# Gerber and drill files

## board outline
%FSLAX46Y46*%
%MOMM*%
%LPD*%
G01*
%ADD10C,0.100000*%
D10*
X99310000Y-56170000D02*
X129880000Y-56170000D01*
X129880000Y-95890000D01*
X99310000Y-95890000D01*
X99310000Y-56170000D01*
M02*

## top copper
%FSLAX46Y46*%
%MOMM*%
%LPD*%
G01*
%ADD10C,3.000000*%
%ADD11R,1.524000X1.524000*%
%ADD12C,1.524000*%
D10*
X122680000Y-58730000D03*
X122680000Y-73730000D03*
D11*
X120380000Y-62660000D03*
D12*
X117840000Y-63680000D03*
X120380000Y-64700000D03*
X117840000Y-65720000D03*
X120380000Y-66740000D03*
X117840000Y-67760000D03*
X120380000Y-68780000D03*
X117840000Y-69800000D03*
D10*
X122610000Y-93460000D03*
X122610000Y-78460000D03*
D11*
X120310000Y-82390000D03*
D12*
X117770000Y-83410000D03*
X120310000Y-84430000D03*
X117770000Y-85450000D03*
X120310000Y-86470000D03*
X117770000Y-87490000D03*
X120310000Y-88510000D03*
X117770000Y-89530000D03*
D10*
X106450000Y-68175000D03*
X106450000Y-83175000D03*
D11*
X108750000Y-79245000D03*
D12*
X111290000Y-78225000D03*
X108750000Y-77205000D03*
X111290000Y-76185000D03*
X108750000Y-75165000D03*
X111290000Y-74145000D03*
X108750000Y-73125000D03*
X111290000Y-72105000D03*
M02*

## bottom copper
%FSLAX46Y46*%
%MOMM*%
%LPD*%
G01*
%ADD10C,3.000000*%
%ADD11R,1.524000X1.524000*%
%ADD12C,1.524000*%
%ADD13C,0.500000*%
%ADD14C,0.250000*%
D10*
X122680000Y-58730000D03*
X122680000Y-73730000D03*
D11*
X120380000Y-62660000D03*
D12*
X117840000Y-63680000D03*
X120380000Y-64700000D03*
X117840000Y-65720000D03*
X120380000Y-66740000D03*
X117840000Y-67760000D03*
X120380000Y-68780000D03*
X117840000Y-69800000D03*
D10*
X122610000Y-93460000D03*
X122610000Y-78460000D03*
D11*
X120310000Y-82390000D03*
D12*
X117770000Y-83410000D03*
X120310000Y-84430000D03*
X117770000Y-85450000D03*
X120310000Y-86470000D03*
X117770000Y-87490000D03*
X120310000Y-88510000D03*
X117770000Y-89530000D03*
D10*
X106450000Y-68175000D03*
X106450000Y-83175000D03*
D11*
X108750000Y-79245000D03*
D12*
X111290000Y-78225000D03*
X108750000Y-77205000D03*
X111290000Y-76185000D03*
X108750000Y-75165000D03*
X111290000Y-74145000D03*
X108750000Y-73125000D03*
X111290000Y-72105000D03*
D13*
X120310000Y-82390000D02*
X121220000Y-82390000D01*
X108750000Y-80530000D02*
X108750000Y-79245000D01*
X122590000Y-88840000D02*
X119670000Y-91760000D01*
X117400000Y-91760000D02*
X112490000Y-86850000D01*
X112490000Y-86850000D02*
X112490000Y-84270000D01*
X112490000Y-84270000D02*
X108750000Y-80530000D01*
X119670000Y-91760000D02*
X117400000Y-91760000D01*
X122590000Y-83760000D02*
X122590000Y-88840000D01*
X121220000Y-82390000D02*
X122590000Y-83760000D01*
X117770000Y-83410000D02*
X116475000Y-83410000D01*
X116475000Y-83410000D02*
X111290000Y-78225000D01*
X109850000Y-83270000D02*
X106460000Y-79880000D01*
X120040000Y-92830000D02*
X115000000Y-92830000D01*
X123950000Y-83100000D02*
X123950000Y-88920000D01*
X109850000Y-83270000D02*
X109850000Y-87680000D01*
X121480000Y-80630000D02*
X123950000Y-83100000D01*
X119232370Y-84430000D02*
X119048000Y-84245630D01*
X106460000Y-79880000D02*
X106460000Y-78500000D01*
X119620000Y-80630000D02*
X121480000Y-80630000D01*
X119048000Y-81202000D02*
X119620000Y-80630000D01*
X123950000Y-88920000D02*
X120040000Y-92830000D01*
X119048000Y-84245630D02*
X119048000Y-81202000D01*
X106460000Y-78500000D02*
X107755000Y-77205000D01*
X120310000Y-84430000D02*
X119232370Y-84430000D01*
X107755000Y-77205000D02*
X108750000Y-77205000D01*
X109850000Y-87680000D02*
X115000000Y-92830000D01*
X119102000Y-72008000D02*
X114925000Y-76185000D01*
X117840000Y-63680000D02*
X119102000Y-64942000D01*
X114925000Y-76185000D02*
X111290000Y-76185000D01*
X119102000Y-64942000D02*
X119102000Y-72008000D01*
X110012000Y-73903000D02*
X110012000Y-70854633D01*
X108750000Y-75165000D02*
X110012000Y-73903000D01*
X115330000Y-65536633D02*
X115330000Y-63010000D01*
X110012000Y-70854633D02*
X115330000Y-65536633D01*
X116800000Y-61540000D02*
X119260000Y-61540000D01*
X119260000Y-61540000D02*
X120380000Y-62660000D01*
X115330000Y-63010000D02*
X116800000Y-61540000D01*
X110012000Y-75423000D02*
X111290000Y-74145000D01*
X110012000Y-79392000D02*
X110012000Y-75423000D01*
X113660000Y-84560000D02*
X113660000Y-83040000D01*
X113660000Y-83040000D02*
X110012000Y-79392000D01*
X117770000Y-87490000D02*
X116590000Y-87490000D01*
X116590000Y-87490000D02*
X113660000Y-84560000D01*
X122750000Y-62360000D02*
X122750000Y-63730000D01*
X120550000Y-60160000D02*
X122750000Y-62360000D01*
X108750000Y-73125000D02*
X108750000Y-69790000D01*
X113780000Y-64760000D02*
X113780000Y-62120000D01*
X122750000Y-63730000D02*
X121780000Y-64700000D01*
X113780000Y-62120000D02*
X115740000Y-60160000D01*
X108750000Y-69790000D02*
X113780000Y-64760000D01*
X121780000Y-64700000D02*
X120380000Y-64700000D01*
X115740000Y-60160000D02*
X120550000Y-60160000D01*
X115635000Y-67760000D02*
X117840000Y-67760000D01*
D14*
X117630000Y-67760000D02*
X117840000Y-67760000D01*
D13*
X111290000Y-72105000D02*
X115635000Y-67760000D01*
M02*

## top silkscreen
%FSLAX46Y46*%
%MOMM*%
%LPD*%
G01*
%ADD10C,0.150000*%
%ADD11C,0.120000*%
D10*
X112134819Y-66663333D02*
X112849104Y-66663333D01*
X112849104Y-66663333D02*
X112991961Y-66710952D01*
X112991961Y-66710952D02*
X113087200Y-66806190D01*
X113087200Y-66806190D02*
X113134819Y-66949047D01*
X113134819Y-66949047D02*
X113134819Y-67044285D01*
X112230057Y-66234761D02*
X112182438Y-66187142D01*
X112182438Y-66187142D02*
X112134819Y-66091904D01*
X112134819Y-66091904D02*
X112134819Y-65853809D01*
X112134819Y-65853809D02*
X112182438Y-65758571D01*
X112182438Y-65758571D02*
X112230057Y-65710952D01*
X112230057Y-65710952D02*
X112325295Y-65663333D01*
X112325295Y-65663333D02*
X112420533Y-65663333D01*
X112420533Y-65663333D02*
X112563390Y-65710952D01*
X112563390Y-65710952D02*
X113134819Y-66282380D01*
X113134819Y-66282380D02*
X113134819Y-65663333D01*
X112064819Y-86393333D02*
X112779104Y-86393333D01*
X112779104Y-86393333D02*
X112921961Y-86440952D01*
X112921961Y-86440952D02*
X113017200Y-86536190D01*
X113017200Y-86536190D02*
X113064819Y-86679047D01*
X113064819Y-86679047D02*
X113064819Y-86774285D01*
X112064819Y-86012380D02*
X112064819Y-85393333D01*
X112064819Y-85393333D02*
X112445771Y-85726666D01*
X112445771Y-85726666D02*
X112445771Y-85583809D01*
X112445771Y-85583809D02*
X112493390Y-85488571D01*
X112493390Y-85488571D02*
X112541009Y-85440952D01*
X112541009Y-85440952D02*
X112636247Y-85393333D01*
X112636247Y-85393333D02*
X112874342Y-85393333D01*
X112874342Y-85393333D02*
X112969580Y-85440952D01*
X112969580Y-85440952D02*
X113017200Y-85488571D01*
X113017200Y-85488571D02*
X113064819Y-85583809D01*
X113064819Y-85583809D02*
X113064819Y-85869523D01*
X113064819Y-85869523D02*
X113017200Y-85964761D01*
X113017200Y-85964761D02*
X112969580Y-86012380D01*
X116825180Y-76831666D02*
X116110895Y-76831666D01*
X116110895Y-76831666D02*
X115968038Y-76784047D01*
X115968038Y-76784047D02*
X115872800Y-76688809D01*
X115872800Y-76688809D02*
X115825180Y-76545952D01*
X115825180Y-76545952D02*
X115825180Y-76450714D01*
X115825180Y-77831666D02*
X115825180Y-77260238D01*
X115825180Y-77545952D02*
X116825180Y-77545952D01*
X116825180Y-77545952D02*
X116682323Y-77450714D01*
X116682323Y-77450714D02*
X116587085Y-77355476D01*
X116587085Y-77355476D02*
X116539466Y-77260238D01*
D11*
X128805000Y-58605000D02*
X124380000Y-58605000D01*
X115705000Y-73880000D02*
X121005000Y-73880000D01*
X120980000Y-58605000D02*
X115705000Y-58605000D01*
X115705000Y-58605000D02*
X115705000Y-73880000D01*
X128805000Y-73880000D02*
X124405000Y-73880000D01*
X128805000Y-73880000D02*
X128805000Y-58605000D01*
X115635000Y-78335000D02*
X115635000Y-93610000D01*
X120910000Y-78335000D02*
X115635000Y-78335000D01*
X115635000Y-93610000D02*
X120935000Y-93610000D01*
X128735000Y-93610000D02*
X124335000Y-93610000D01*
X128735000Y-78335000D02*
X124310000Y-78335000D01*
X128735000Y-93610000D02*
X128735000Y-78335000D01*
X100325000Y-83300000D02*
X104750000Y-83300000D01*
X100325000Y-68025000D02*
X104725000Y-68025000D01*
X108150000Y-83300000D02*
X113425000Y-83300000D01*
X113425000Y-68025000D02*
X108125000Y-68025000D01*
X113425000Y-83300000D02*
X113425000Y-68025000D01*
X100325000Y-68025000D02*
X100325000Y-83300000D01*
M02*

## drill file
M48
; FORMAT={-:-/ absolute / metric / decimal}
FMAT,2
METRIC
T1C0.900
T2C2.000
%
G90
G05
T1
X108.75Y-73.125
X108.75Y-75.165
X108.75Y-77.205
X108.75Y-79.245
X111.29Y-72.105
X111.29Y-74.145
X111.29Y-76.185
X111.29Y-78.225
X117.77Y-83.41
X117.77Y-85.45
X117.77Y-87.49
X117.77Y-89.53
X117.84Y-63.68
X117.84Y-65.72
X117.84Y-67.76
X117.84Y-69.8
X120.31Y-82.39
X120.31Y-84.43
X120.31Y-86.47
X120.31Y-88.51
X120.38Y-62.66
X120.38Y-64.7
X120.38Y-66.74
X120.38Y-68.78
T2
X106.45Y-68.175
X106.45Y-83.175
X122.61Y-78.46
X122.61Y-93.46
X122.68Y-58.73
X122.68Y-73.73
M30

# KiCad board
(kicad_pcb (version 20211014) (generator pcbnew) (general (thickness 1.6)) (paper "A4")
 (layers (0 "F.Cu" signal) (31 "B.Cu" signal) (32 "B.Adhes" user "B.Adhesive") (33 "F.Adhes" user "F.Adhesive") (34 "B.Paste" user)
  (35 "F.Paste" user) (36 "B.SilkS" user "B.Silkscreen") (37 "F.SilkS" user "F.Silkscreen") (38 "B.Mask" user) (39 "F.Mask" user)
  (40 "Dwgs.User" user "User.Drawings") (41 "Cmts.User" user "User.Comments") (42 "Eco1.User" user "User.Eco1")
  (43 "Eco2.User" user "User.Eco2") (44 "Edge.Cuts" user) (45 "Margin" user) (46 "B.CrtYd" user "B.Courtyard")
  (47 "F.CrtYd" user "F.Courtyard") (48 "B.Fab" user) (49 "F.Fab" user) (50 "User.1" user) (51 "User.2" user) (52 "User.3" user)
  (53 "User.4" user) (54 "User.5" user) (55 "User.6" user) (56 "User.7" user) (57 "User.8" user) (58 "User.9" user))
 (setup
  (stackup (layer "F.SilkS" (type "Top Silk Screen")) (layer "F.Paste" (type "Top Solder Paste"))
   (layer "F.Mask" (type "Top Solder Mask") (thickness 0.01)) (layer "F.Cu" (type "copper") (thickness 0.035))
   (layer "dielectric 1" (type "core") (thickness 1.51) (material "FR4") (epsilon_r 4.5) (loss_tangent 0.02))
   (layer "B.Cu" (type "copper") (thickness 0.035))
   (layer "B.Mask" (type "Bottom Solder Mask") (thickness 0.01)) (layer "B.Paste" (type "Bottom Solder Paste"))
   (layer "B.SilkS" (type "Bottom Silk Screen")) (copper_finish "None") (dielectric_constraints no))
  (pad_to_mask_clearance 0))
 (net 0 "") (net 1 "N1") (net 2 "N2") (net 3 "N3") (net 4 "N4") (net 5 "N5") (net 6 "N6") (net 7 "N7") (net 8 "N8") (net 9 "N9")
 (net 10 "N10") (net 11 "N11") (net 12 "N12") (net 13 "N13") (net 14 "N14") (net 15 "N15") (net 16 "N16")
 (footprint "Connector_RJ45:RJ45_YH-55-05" (layer "F.Cu") (at 122.68 73.73 90)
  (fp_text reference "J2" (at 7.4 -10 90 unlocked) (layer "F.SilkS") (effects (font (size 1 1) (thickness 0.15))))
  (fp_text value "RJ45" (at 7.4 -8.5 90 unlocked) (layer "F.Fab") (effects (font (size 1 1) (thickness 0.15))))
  (fp_line (start 15.125 6.125) (end 15.125 1.7) (layer "F.SilkS") (width 0.12))
  (fp_line (start -0.15 -6.975) (end -0.15 -1.675) (layer "F.SilkS") (width 0.12))
  (fp_line (start 15.125 -1.7) (end 15.125 -6.975) (layer "F.SilkS") (width 0.12))
  (fp_line (start 15.125 -6.975) (end -0.15 -6.975) (layer "F.SilkS") (width 0.12))
  (fp_line (start -0.15 6.125) (end -0.15 1.725) (layer "F.SilkS") (width 0.12))
  (fp_line (start -0.15 6.125) (end 15.125 6.125) (layer "F.SilkS") (width 0.12))
  (pad "" np_thru_hole circle (at 15 0 90) (size 3 3) (drill 2) (layers F&B.Cu *.Mask))
  (pad "" np_thru_hole circle (at 0 0 90) (size 3 3) (drill 2) (layers F&B.Cu *.Mask))
  (pad "1" thru_hole rect (at 11.07 -2.3 90) (size 1.524 1.524) (drill 0.9) (layers *.Cu *.Mask) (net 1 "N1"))
  (pad "2" thru_hole circle (at 10.05 -4.84 90) (size 1.524 1.524) (drill 0.9) (layers *.Cu *.Mask) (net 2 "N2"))
  (pad "3" thru_hole circle (at 9.03 -2.3 90) (size 1.524 1.524) (drill 0.9) (layers *.Cu *.Mask) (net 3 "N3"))
  (pad "4" thru_hole circle (at 8.01 -4.84 90) (size 1.524 1.524) (drill 0.9) (layers *.Cu *.Mask) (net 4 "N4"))
  (pad "5" thru_hole circle (at 6.99 -2.3 90) (size 1.524 1.524) (drill 0.9) (layers *.Cu *.Mask) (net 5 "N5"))
  (pad "6" thru_hole circle (at 5.97 -4.84 90) (size 1.524 1.524) (drill 0.9) (layers *.Cu *.Mask) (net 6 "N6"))
  (pad "7" thru_hole circle (at 4.95 -2.3 90) (size 1.524 1.524) (drill 0.9) (layers *.Cu *.Mask) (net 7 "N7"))
  (pad "8" thru_hole circle (at 3.93 -4.84 90) (size 1.524 1.524) (drill 0.9) (layers *.Cu *.Mask) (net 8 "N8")))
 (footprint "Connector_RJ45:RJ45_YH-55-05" (layer "F.Cu") (at 122.61 93.46 90)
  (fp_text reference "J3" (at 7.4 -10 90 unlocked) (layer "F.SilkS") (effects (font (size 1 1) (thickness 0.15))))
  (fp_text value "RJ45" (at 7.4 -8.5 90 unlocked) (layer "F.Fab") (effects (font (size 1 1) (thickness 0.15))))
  (fp_line (start 15.125 -6.975) (end -0.15 -6.975) (layer "F.SilkS") (width 0.12))
  (fp_line (start 15.125 -1.7) (end 15.125 -6.975) (layer "F.SilkS") (width 0.12))
  (fp_line (start -0.15 -6.975) (end -0.15 -1.675) (layer "F.SilkS") (width 0.12))
  (fp_line (start -0.15 6.125) (end -0.15 1.725) (layer "F.SilkS") (width 0.12))
  (fp_line (start 15.125 6.125) (end 15.125 1.7) (layer "F.SilkS") (width 0.12))
  (fp_line (start -0.15 6.125) (end 15.125 6.125) (layer "F.SilkS") (width 0.12))
  (pad "" np_thru_hole circle (at 0 0 90) (size 3 3) (drill 2) (layers F&B.Cu *.Mask))
  (pad "" np_thru_hole circle (at 15 0 90) (size 3 3) (drill 2) (layers F&B.Cu *.Mask))
  (pad "1" thru_hole rect (at 11.07 -2.3 90) (size 1.524 1.524) (drill 0.9) (layers *.Cu *.Mask) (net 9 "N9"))
  (pad "2" thru_hole circle (at 10.05 -4.84 90) (size 1.524 1.524) (drill 0.9) (layers *.Cu *.Mask) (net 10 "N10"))
  (pad "3" thru_hole circle (at 9.03 -2.3 90) (size 1.524 1.524) (drill 0.9) (layers *.Cu *.Mask) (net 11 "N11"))
  (pad "4" thru_hole circle (at 8.01 -4.84 90) (size 1.524 1.524) (drill 0.9) (layers *.Cu *.Mask) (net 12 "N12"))
  (pad "5" thru_hole circle (at 6.99 -2.3 90) (size 1.524 1.524) (drill 0.9) (layers *.Cu *.Mask) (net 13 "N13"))
  (pad "6" thru_hole circle (at 5.97 -4.84 90) (size 1.524 1.524) (drill 0.9) (layers *.Cu *.Mask) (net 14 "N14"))
  (pad "7" thru_hole circle (at 4.95 -2.3 90) (size 1.524 1.524) (drill 0.9) (layers *.Cu *.Mask) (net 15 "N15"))
  (pad "8" thru_hole circle (at 3.93 -4.84 90) (size 1.524 1.524) (drill 0.9) (layers *.Cu *.Mask) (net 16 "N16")))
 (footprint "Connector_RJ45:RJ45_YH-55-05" (layer "F.Cu") (at 106.45 68.175 -90)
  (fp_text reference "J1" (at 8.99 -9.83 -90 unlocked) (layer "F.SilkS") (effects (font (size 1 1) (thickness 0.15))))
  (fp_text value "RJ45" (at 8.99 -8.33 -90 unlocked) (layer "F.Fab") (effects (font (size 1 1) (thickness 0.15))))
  (fp_line (start 15.125 6.125) (end 15.125 1.7) (layer "F.SilkS") (width 0.12))
  (fp_line (start -0.15 6.125) (end -0.15 1.725) (layer "F.SilkS") (width 0.12))
  (fp_line (start 15.125 -1.7) (end 15.125 -6.975) (layer "F.SilkS") (width 0.12))
  (fp_line (start -0.15 -6.975) (end -0.15 -1.675) (layer "F.SilkS") (width 0.12))
  (fp_line (start 15.125 -6.975) (end -0.15 -6.975) (layer "F.SilkS") (width 0.12))
  (fp_line (start -0.15 6.125) (end 15.125 6.125) (layer "F.SilkS") (width 0.12))
  (pad "" np_thru_hole circle (at 0 0 270) (size 3 3) (drill 2) (layers F&B.Cu *.Mask))
  (pad "" np_thru_hole circle (at 15 0 270) (size 3 3) (drill 2) (layers F&B.Cu *.Mask))
  (pad "1" thru_hole rect (at 11.07 -2.3 270) (size 1.524 1.524) (drill 0.9) (layers *.Cu *.Mask) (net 9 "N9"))
  (pad "2" thru_hole circle (at 10.05 -4.84 270) (size 1.524 1.524) (drill 0.9) (layers *.Cu *.Mask) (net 10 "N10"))
  (pad "3" thru_hole circle (at 9.03 -2.3 270) (size 1.524 1.524) (drill 0.9) (layers *.Cu *.Mask) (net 11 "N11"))
  (pad "4" thru_hole circle (at 8.01 -4.84 270) (size 1.524 1.524) (drill 0.9) (layers *.Cu *.Mask) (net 2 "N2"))
  (pad "5" thru_hole circle (at 6.99 -2.3 270) (size 1.524 1.524) (drill 0.9) (layers *.Cu *.Mask) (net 1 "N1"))
  (pad "6" thru_hole circle (at 5.97 -4.84 270) (size 1.524 1.524) (drill 0.9) (layers *.Cu *.Mask) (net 14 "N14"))
  (pad "7" thru_hole circle (at 4.95 -2.3 270) (size 1.524 1.524) (drill 0.9) (layers *.Cu *.Mask) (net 3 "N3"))
  (pad "8" thru_hole circle (at 3.93 -4.84 270) (size 1.524 1.524) (drill 0.9) (layers *.Cu *.Mask) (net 6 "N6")))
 (gr_rect (start 129.88 56.17) (end 99.31 95.89) (layer "Edge.Cuts") (width 0.1) (fill none))
 (segment (start 120.31 82.39) (end 121.22 82.39) (width 0.5) (layer "B.Cu") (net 9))
 (segment (start 108.75 80.53) (end 108.75 79.245) (width 0.5) (layer "B.Cu") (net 9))
 (segment (start 122.59 88.84) (end 119.67 91.76) (width 0.5) (layer "B.Cu") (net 9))
 (segment (start 117.4 91.76) (end 112.49 86.85) (width 0.5) (layer "B.Cu") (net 9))
 (segment (start 112.49 86.85) (end 112.49 84.27) (width 0.5) (layer "B.Cu") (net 9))
 (segment (start 112.49 84.27) (end 108.75 80.53) (width 0.5) (layer "B.Cu") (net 9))
 (segment (start 119.67 91.76) (end 117.4 91.76) (width 0.5) (layer "B.Cu") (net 9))
 (segment (start 122.59 83.76) (end 122.59 88.84) (width 0.5) (layer "B.Cu") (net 9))
 (segment (start 121.22 82.39) (end 122.59 83.76) (width 0.5) (layer "B.Cu") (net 9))
 (segment (start 117.77 83.41) (end 116.475 83.41) (width 0.5) (layer "B.Cu") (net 10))
 (segment (start 116.475 83.41) (end 111.29 78.225) (width 0.5) (layer "B.Cu") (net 10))
 (segment (start 109.85 83.27) (end 106.46 79.88) (width 0.5) (layer "B.Cu") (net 11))
 (segment (start 120.04 92.83) (end 115 92.83) (width 0.5) (layer "B.Cu") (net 11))
 (segment (start 123.95 83.1) (end 123.95 88.92) (width 0.5) (layer "B.Cu") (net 11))
 (segment (start 109.85 83.27) (end 109.85 87.68) (width 0.5) (layer "B.Cu") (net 11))
 (segment (start 121.48 80.63) (end 123.95 83.1) (width 0.5) (layer "B.Cu") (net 11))
 (segment (start 119.23237 84.43) (end 119.048 84.24563) (width 0.5) (layer "B.Cu") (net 11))
 (segment (start 106.46 79.88) (end 106.46 78.5) (width 0.5) (layer "B.Cu") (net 11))
 (segment (start 119.62 80.63) (end 121.48 80.63) (width 0.5) (layer "B.Cu") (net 11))
 (segment (start 119.048 81.202) (end 119.62 80.63) (width 0.5) (layer "B.Cu") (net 11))
 (segment (start 123.95 88.92) (end 120.04 92.83) (width 0.5) (layer "B.Cu") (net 11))
 (segment (start 119.048 84.24563) (end 119.048 81.202) (width 0.5) (layer "B.Cu") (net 11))
 (segment (start 106.46 78.5) (end 107.755 77.205) (width 0.5) (layer "B.Cu") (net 11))
 (segment (start 120.31 84.43) (end 119.23237 84.43) (width 0.5) (layer "B.Cu") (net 11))
 (segment (start 107.755 77.205) (end 108.75 77.205) (width 0.5) (layer "B.Cu") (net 11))
 (segment (start 109.85 87.68) (end 115 92.83) (width 0.5) (layer "B.Cu") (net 11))
 (segment (start 119.102 72.008) (end 114.925 76.185) (width 0.5) (layer "B.Cu") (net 2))
 (segment (start 117.84 63.68) (end 119.102 64.942) (width 0.5) (layer "B.Cu") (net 2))
 (segment (start 114.925 76.185) (end 111.29 76.185) (width 0.5) (layer "B.Cu") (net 2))
 (segment (start 119.102 64.942) (end 119.102 72.008) (width 0.5) (layer "B.Cu") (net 2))
 (segment (start 110.012 73.903) (end 110.012 70.854633) (width 0.5) (layer "B.Cu") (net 1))
 (segment (start 108.75 75.165) (end 110.012 73.903) (width 0.5) (layer "B.Cu") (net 1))
 (segment (start 115.33 65.536633) (end 115.33 63.01) (width 0.5) (layer "B.Cu") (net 1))
 (segment (start 110.012 70.854633) (end 115.33 65.536633) (width 0.5) (layer "B.Cu") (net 1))
 (segment (start 116.8 61.54) (end 119.26 61.54) (width 0.5) (layer "B.Cu") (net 1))
 (segment (start 119.26 61.54) (end 120.38 62.66) (width 0.5) (layer "B.Cu") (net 1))
 (segment (start 115.33 63.01) (end 116.8 61.54) (width 0.5) (layer "B.Cu") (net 1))
 (segment (start 110.012 75.423) (end 111.29 74.145) (width 0.5) (layer "B.Cu") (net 14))
 (segment (start 110.012 79.392) (end 110.012 75.423) (width 0.5) (layer "B.Cu") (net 14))
 (segment (start 113.66 84.56) (end 113.66 83.04) (width 0.5) (layer "B.Cu") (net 14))
 (segment (start 113.66 83.04) (end 110.012 79.392) (width 0.5) (layer "B.Cu") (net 14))
 (segment (start 117.77 87.49) (end 116.59 87.49) (width 0.5) (layer "B.Cu") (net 14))
 (segment (start 116.59 87.49) (end 113.66 84.56) (width 0.5) (layer "B.Cu") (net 14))
 (segment (start 122.75 62.36) (end 122.75 63.73) (width 0.5) (layer "B.Cu") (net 3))
 (segment (start 120.55 60.16) (end 122.75 62.36) (width 0.5) (layer "B.Cu") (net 3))
 (segment (start 108.75 73.125) (end 108.75 69.79) (width 0.5) (layer "B.Cu") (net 3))
 (segment (start 113.78 64.76) (end 113.78 62.12) (width 0.5) (layer "B.Cu") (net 3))
 (segment (start 122.75 63.73) (end 121.78 64.7) (width 0.5) (layer "B.Cu") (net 3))
 (segment (start 113.78 62.12) (end 115.74 60.16) (width 0.5) (layer "B.Cu") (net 3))
 (segment (start 108.75 69.79) (end 113.78 64.76) (width 0.5) (layer "B.Cu") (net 3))
 (segment (start 121.78 64.7) (end 120.38 64.7) (width 0.5) (layer "B.Cu") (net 3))
 (segment (start 115.74 60.16) (end 120.55 60.16) (width 0.5) (layer "B.Cu") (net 3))
 (segment (start 115.635 67.76) (end 117.84 67.76) (width 0.5) (layer "B.Cu") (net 6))
 (segment (start 117.63 67.76) (end 117.84 67.76) (width 0.25) (layer "B.Cu") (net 6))
 (segment (start 111.29 72.105) (end 115.635 67.76) (width 0.5) (layer "B.Cu") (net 6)))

